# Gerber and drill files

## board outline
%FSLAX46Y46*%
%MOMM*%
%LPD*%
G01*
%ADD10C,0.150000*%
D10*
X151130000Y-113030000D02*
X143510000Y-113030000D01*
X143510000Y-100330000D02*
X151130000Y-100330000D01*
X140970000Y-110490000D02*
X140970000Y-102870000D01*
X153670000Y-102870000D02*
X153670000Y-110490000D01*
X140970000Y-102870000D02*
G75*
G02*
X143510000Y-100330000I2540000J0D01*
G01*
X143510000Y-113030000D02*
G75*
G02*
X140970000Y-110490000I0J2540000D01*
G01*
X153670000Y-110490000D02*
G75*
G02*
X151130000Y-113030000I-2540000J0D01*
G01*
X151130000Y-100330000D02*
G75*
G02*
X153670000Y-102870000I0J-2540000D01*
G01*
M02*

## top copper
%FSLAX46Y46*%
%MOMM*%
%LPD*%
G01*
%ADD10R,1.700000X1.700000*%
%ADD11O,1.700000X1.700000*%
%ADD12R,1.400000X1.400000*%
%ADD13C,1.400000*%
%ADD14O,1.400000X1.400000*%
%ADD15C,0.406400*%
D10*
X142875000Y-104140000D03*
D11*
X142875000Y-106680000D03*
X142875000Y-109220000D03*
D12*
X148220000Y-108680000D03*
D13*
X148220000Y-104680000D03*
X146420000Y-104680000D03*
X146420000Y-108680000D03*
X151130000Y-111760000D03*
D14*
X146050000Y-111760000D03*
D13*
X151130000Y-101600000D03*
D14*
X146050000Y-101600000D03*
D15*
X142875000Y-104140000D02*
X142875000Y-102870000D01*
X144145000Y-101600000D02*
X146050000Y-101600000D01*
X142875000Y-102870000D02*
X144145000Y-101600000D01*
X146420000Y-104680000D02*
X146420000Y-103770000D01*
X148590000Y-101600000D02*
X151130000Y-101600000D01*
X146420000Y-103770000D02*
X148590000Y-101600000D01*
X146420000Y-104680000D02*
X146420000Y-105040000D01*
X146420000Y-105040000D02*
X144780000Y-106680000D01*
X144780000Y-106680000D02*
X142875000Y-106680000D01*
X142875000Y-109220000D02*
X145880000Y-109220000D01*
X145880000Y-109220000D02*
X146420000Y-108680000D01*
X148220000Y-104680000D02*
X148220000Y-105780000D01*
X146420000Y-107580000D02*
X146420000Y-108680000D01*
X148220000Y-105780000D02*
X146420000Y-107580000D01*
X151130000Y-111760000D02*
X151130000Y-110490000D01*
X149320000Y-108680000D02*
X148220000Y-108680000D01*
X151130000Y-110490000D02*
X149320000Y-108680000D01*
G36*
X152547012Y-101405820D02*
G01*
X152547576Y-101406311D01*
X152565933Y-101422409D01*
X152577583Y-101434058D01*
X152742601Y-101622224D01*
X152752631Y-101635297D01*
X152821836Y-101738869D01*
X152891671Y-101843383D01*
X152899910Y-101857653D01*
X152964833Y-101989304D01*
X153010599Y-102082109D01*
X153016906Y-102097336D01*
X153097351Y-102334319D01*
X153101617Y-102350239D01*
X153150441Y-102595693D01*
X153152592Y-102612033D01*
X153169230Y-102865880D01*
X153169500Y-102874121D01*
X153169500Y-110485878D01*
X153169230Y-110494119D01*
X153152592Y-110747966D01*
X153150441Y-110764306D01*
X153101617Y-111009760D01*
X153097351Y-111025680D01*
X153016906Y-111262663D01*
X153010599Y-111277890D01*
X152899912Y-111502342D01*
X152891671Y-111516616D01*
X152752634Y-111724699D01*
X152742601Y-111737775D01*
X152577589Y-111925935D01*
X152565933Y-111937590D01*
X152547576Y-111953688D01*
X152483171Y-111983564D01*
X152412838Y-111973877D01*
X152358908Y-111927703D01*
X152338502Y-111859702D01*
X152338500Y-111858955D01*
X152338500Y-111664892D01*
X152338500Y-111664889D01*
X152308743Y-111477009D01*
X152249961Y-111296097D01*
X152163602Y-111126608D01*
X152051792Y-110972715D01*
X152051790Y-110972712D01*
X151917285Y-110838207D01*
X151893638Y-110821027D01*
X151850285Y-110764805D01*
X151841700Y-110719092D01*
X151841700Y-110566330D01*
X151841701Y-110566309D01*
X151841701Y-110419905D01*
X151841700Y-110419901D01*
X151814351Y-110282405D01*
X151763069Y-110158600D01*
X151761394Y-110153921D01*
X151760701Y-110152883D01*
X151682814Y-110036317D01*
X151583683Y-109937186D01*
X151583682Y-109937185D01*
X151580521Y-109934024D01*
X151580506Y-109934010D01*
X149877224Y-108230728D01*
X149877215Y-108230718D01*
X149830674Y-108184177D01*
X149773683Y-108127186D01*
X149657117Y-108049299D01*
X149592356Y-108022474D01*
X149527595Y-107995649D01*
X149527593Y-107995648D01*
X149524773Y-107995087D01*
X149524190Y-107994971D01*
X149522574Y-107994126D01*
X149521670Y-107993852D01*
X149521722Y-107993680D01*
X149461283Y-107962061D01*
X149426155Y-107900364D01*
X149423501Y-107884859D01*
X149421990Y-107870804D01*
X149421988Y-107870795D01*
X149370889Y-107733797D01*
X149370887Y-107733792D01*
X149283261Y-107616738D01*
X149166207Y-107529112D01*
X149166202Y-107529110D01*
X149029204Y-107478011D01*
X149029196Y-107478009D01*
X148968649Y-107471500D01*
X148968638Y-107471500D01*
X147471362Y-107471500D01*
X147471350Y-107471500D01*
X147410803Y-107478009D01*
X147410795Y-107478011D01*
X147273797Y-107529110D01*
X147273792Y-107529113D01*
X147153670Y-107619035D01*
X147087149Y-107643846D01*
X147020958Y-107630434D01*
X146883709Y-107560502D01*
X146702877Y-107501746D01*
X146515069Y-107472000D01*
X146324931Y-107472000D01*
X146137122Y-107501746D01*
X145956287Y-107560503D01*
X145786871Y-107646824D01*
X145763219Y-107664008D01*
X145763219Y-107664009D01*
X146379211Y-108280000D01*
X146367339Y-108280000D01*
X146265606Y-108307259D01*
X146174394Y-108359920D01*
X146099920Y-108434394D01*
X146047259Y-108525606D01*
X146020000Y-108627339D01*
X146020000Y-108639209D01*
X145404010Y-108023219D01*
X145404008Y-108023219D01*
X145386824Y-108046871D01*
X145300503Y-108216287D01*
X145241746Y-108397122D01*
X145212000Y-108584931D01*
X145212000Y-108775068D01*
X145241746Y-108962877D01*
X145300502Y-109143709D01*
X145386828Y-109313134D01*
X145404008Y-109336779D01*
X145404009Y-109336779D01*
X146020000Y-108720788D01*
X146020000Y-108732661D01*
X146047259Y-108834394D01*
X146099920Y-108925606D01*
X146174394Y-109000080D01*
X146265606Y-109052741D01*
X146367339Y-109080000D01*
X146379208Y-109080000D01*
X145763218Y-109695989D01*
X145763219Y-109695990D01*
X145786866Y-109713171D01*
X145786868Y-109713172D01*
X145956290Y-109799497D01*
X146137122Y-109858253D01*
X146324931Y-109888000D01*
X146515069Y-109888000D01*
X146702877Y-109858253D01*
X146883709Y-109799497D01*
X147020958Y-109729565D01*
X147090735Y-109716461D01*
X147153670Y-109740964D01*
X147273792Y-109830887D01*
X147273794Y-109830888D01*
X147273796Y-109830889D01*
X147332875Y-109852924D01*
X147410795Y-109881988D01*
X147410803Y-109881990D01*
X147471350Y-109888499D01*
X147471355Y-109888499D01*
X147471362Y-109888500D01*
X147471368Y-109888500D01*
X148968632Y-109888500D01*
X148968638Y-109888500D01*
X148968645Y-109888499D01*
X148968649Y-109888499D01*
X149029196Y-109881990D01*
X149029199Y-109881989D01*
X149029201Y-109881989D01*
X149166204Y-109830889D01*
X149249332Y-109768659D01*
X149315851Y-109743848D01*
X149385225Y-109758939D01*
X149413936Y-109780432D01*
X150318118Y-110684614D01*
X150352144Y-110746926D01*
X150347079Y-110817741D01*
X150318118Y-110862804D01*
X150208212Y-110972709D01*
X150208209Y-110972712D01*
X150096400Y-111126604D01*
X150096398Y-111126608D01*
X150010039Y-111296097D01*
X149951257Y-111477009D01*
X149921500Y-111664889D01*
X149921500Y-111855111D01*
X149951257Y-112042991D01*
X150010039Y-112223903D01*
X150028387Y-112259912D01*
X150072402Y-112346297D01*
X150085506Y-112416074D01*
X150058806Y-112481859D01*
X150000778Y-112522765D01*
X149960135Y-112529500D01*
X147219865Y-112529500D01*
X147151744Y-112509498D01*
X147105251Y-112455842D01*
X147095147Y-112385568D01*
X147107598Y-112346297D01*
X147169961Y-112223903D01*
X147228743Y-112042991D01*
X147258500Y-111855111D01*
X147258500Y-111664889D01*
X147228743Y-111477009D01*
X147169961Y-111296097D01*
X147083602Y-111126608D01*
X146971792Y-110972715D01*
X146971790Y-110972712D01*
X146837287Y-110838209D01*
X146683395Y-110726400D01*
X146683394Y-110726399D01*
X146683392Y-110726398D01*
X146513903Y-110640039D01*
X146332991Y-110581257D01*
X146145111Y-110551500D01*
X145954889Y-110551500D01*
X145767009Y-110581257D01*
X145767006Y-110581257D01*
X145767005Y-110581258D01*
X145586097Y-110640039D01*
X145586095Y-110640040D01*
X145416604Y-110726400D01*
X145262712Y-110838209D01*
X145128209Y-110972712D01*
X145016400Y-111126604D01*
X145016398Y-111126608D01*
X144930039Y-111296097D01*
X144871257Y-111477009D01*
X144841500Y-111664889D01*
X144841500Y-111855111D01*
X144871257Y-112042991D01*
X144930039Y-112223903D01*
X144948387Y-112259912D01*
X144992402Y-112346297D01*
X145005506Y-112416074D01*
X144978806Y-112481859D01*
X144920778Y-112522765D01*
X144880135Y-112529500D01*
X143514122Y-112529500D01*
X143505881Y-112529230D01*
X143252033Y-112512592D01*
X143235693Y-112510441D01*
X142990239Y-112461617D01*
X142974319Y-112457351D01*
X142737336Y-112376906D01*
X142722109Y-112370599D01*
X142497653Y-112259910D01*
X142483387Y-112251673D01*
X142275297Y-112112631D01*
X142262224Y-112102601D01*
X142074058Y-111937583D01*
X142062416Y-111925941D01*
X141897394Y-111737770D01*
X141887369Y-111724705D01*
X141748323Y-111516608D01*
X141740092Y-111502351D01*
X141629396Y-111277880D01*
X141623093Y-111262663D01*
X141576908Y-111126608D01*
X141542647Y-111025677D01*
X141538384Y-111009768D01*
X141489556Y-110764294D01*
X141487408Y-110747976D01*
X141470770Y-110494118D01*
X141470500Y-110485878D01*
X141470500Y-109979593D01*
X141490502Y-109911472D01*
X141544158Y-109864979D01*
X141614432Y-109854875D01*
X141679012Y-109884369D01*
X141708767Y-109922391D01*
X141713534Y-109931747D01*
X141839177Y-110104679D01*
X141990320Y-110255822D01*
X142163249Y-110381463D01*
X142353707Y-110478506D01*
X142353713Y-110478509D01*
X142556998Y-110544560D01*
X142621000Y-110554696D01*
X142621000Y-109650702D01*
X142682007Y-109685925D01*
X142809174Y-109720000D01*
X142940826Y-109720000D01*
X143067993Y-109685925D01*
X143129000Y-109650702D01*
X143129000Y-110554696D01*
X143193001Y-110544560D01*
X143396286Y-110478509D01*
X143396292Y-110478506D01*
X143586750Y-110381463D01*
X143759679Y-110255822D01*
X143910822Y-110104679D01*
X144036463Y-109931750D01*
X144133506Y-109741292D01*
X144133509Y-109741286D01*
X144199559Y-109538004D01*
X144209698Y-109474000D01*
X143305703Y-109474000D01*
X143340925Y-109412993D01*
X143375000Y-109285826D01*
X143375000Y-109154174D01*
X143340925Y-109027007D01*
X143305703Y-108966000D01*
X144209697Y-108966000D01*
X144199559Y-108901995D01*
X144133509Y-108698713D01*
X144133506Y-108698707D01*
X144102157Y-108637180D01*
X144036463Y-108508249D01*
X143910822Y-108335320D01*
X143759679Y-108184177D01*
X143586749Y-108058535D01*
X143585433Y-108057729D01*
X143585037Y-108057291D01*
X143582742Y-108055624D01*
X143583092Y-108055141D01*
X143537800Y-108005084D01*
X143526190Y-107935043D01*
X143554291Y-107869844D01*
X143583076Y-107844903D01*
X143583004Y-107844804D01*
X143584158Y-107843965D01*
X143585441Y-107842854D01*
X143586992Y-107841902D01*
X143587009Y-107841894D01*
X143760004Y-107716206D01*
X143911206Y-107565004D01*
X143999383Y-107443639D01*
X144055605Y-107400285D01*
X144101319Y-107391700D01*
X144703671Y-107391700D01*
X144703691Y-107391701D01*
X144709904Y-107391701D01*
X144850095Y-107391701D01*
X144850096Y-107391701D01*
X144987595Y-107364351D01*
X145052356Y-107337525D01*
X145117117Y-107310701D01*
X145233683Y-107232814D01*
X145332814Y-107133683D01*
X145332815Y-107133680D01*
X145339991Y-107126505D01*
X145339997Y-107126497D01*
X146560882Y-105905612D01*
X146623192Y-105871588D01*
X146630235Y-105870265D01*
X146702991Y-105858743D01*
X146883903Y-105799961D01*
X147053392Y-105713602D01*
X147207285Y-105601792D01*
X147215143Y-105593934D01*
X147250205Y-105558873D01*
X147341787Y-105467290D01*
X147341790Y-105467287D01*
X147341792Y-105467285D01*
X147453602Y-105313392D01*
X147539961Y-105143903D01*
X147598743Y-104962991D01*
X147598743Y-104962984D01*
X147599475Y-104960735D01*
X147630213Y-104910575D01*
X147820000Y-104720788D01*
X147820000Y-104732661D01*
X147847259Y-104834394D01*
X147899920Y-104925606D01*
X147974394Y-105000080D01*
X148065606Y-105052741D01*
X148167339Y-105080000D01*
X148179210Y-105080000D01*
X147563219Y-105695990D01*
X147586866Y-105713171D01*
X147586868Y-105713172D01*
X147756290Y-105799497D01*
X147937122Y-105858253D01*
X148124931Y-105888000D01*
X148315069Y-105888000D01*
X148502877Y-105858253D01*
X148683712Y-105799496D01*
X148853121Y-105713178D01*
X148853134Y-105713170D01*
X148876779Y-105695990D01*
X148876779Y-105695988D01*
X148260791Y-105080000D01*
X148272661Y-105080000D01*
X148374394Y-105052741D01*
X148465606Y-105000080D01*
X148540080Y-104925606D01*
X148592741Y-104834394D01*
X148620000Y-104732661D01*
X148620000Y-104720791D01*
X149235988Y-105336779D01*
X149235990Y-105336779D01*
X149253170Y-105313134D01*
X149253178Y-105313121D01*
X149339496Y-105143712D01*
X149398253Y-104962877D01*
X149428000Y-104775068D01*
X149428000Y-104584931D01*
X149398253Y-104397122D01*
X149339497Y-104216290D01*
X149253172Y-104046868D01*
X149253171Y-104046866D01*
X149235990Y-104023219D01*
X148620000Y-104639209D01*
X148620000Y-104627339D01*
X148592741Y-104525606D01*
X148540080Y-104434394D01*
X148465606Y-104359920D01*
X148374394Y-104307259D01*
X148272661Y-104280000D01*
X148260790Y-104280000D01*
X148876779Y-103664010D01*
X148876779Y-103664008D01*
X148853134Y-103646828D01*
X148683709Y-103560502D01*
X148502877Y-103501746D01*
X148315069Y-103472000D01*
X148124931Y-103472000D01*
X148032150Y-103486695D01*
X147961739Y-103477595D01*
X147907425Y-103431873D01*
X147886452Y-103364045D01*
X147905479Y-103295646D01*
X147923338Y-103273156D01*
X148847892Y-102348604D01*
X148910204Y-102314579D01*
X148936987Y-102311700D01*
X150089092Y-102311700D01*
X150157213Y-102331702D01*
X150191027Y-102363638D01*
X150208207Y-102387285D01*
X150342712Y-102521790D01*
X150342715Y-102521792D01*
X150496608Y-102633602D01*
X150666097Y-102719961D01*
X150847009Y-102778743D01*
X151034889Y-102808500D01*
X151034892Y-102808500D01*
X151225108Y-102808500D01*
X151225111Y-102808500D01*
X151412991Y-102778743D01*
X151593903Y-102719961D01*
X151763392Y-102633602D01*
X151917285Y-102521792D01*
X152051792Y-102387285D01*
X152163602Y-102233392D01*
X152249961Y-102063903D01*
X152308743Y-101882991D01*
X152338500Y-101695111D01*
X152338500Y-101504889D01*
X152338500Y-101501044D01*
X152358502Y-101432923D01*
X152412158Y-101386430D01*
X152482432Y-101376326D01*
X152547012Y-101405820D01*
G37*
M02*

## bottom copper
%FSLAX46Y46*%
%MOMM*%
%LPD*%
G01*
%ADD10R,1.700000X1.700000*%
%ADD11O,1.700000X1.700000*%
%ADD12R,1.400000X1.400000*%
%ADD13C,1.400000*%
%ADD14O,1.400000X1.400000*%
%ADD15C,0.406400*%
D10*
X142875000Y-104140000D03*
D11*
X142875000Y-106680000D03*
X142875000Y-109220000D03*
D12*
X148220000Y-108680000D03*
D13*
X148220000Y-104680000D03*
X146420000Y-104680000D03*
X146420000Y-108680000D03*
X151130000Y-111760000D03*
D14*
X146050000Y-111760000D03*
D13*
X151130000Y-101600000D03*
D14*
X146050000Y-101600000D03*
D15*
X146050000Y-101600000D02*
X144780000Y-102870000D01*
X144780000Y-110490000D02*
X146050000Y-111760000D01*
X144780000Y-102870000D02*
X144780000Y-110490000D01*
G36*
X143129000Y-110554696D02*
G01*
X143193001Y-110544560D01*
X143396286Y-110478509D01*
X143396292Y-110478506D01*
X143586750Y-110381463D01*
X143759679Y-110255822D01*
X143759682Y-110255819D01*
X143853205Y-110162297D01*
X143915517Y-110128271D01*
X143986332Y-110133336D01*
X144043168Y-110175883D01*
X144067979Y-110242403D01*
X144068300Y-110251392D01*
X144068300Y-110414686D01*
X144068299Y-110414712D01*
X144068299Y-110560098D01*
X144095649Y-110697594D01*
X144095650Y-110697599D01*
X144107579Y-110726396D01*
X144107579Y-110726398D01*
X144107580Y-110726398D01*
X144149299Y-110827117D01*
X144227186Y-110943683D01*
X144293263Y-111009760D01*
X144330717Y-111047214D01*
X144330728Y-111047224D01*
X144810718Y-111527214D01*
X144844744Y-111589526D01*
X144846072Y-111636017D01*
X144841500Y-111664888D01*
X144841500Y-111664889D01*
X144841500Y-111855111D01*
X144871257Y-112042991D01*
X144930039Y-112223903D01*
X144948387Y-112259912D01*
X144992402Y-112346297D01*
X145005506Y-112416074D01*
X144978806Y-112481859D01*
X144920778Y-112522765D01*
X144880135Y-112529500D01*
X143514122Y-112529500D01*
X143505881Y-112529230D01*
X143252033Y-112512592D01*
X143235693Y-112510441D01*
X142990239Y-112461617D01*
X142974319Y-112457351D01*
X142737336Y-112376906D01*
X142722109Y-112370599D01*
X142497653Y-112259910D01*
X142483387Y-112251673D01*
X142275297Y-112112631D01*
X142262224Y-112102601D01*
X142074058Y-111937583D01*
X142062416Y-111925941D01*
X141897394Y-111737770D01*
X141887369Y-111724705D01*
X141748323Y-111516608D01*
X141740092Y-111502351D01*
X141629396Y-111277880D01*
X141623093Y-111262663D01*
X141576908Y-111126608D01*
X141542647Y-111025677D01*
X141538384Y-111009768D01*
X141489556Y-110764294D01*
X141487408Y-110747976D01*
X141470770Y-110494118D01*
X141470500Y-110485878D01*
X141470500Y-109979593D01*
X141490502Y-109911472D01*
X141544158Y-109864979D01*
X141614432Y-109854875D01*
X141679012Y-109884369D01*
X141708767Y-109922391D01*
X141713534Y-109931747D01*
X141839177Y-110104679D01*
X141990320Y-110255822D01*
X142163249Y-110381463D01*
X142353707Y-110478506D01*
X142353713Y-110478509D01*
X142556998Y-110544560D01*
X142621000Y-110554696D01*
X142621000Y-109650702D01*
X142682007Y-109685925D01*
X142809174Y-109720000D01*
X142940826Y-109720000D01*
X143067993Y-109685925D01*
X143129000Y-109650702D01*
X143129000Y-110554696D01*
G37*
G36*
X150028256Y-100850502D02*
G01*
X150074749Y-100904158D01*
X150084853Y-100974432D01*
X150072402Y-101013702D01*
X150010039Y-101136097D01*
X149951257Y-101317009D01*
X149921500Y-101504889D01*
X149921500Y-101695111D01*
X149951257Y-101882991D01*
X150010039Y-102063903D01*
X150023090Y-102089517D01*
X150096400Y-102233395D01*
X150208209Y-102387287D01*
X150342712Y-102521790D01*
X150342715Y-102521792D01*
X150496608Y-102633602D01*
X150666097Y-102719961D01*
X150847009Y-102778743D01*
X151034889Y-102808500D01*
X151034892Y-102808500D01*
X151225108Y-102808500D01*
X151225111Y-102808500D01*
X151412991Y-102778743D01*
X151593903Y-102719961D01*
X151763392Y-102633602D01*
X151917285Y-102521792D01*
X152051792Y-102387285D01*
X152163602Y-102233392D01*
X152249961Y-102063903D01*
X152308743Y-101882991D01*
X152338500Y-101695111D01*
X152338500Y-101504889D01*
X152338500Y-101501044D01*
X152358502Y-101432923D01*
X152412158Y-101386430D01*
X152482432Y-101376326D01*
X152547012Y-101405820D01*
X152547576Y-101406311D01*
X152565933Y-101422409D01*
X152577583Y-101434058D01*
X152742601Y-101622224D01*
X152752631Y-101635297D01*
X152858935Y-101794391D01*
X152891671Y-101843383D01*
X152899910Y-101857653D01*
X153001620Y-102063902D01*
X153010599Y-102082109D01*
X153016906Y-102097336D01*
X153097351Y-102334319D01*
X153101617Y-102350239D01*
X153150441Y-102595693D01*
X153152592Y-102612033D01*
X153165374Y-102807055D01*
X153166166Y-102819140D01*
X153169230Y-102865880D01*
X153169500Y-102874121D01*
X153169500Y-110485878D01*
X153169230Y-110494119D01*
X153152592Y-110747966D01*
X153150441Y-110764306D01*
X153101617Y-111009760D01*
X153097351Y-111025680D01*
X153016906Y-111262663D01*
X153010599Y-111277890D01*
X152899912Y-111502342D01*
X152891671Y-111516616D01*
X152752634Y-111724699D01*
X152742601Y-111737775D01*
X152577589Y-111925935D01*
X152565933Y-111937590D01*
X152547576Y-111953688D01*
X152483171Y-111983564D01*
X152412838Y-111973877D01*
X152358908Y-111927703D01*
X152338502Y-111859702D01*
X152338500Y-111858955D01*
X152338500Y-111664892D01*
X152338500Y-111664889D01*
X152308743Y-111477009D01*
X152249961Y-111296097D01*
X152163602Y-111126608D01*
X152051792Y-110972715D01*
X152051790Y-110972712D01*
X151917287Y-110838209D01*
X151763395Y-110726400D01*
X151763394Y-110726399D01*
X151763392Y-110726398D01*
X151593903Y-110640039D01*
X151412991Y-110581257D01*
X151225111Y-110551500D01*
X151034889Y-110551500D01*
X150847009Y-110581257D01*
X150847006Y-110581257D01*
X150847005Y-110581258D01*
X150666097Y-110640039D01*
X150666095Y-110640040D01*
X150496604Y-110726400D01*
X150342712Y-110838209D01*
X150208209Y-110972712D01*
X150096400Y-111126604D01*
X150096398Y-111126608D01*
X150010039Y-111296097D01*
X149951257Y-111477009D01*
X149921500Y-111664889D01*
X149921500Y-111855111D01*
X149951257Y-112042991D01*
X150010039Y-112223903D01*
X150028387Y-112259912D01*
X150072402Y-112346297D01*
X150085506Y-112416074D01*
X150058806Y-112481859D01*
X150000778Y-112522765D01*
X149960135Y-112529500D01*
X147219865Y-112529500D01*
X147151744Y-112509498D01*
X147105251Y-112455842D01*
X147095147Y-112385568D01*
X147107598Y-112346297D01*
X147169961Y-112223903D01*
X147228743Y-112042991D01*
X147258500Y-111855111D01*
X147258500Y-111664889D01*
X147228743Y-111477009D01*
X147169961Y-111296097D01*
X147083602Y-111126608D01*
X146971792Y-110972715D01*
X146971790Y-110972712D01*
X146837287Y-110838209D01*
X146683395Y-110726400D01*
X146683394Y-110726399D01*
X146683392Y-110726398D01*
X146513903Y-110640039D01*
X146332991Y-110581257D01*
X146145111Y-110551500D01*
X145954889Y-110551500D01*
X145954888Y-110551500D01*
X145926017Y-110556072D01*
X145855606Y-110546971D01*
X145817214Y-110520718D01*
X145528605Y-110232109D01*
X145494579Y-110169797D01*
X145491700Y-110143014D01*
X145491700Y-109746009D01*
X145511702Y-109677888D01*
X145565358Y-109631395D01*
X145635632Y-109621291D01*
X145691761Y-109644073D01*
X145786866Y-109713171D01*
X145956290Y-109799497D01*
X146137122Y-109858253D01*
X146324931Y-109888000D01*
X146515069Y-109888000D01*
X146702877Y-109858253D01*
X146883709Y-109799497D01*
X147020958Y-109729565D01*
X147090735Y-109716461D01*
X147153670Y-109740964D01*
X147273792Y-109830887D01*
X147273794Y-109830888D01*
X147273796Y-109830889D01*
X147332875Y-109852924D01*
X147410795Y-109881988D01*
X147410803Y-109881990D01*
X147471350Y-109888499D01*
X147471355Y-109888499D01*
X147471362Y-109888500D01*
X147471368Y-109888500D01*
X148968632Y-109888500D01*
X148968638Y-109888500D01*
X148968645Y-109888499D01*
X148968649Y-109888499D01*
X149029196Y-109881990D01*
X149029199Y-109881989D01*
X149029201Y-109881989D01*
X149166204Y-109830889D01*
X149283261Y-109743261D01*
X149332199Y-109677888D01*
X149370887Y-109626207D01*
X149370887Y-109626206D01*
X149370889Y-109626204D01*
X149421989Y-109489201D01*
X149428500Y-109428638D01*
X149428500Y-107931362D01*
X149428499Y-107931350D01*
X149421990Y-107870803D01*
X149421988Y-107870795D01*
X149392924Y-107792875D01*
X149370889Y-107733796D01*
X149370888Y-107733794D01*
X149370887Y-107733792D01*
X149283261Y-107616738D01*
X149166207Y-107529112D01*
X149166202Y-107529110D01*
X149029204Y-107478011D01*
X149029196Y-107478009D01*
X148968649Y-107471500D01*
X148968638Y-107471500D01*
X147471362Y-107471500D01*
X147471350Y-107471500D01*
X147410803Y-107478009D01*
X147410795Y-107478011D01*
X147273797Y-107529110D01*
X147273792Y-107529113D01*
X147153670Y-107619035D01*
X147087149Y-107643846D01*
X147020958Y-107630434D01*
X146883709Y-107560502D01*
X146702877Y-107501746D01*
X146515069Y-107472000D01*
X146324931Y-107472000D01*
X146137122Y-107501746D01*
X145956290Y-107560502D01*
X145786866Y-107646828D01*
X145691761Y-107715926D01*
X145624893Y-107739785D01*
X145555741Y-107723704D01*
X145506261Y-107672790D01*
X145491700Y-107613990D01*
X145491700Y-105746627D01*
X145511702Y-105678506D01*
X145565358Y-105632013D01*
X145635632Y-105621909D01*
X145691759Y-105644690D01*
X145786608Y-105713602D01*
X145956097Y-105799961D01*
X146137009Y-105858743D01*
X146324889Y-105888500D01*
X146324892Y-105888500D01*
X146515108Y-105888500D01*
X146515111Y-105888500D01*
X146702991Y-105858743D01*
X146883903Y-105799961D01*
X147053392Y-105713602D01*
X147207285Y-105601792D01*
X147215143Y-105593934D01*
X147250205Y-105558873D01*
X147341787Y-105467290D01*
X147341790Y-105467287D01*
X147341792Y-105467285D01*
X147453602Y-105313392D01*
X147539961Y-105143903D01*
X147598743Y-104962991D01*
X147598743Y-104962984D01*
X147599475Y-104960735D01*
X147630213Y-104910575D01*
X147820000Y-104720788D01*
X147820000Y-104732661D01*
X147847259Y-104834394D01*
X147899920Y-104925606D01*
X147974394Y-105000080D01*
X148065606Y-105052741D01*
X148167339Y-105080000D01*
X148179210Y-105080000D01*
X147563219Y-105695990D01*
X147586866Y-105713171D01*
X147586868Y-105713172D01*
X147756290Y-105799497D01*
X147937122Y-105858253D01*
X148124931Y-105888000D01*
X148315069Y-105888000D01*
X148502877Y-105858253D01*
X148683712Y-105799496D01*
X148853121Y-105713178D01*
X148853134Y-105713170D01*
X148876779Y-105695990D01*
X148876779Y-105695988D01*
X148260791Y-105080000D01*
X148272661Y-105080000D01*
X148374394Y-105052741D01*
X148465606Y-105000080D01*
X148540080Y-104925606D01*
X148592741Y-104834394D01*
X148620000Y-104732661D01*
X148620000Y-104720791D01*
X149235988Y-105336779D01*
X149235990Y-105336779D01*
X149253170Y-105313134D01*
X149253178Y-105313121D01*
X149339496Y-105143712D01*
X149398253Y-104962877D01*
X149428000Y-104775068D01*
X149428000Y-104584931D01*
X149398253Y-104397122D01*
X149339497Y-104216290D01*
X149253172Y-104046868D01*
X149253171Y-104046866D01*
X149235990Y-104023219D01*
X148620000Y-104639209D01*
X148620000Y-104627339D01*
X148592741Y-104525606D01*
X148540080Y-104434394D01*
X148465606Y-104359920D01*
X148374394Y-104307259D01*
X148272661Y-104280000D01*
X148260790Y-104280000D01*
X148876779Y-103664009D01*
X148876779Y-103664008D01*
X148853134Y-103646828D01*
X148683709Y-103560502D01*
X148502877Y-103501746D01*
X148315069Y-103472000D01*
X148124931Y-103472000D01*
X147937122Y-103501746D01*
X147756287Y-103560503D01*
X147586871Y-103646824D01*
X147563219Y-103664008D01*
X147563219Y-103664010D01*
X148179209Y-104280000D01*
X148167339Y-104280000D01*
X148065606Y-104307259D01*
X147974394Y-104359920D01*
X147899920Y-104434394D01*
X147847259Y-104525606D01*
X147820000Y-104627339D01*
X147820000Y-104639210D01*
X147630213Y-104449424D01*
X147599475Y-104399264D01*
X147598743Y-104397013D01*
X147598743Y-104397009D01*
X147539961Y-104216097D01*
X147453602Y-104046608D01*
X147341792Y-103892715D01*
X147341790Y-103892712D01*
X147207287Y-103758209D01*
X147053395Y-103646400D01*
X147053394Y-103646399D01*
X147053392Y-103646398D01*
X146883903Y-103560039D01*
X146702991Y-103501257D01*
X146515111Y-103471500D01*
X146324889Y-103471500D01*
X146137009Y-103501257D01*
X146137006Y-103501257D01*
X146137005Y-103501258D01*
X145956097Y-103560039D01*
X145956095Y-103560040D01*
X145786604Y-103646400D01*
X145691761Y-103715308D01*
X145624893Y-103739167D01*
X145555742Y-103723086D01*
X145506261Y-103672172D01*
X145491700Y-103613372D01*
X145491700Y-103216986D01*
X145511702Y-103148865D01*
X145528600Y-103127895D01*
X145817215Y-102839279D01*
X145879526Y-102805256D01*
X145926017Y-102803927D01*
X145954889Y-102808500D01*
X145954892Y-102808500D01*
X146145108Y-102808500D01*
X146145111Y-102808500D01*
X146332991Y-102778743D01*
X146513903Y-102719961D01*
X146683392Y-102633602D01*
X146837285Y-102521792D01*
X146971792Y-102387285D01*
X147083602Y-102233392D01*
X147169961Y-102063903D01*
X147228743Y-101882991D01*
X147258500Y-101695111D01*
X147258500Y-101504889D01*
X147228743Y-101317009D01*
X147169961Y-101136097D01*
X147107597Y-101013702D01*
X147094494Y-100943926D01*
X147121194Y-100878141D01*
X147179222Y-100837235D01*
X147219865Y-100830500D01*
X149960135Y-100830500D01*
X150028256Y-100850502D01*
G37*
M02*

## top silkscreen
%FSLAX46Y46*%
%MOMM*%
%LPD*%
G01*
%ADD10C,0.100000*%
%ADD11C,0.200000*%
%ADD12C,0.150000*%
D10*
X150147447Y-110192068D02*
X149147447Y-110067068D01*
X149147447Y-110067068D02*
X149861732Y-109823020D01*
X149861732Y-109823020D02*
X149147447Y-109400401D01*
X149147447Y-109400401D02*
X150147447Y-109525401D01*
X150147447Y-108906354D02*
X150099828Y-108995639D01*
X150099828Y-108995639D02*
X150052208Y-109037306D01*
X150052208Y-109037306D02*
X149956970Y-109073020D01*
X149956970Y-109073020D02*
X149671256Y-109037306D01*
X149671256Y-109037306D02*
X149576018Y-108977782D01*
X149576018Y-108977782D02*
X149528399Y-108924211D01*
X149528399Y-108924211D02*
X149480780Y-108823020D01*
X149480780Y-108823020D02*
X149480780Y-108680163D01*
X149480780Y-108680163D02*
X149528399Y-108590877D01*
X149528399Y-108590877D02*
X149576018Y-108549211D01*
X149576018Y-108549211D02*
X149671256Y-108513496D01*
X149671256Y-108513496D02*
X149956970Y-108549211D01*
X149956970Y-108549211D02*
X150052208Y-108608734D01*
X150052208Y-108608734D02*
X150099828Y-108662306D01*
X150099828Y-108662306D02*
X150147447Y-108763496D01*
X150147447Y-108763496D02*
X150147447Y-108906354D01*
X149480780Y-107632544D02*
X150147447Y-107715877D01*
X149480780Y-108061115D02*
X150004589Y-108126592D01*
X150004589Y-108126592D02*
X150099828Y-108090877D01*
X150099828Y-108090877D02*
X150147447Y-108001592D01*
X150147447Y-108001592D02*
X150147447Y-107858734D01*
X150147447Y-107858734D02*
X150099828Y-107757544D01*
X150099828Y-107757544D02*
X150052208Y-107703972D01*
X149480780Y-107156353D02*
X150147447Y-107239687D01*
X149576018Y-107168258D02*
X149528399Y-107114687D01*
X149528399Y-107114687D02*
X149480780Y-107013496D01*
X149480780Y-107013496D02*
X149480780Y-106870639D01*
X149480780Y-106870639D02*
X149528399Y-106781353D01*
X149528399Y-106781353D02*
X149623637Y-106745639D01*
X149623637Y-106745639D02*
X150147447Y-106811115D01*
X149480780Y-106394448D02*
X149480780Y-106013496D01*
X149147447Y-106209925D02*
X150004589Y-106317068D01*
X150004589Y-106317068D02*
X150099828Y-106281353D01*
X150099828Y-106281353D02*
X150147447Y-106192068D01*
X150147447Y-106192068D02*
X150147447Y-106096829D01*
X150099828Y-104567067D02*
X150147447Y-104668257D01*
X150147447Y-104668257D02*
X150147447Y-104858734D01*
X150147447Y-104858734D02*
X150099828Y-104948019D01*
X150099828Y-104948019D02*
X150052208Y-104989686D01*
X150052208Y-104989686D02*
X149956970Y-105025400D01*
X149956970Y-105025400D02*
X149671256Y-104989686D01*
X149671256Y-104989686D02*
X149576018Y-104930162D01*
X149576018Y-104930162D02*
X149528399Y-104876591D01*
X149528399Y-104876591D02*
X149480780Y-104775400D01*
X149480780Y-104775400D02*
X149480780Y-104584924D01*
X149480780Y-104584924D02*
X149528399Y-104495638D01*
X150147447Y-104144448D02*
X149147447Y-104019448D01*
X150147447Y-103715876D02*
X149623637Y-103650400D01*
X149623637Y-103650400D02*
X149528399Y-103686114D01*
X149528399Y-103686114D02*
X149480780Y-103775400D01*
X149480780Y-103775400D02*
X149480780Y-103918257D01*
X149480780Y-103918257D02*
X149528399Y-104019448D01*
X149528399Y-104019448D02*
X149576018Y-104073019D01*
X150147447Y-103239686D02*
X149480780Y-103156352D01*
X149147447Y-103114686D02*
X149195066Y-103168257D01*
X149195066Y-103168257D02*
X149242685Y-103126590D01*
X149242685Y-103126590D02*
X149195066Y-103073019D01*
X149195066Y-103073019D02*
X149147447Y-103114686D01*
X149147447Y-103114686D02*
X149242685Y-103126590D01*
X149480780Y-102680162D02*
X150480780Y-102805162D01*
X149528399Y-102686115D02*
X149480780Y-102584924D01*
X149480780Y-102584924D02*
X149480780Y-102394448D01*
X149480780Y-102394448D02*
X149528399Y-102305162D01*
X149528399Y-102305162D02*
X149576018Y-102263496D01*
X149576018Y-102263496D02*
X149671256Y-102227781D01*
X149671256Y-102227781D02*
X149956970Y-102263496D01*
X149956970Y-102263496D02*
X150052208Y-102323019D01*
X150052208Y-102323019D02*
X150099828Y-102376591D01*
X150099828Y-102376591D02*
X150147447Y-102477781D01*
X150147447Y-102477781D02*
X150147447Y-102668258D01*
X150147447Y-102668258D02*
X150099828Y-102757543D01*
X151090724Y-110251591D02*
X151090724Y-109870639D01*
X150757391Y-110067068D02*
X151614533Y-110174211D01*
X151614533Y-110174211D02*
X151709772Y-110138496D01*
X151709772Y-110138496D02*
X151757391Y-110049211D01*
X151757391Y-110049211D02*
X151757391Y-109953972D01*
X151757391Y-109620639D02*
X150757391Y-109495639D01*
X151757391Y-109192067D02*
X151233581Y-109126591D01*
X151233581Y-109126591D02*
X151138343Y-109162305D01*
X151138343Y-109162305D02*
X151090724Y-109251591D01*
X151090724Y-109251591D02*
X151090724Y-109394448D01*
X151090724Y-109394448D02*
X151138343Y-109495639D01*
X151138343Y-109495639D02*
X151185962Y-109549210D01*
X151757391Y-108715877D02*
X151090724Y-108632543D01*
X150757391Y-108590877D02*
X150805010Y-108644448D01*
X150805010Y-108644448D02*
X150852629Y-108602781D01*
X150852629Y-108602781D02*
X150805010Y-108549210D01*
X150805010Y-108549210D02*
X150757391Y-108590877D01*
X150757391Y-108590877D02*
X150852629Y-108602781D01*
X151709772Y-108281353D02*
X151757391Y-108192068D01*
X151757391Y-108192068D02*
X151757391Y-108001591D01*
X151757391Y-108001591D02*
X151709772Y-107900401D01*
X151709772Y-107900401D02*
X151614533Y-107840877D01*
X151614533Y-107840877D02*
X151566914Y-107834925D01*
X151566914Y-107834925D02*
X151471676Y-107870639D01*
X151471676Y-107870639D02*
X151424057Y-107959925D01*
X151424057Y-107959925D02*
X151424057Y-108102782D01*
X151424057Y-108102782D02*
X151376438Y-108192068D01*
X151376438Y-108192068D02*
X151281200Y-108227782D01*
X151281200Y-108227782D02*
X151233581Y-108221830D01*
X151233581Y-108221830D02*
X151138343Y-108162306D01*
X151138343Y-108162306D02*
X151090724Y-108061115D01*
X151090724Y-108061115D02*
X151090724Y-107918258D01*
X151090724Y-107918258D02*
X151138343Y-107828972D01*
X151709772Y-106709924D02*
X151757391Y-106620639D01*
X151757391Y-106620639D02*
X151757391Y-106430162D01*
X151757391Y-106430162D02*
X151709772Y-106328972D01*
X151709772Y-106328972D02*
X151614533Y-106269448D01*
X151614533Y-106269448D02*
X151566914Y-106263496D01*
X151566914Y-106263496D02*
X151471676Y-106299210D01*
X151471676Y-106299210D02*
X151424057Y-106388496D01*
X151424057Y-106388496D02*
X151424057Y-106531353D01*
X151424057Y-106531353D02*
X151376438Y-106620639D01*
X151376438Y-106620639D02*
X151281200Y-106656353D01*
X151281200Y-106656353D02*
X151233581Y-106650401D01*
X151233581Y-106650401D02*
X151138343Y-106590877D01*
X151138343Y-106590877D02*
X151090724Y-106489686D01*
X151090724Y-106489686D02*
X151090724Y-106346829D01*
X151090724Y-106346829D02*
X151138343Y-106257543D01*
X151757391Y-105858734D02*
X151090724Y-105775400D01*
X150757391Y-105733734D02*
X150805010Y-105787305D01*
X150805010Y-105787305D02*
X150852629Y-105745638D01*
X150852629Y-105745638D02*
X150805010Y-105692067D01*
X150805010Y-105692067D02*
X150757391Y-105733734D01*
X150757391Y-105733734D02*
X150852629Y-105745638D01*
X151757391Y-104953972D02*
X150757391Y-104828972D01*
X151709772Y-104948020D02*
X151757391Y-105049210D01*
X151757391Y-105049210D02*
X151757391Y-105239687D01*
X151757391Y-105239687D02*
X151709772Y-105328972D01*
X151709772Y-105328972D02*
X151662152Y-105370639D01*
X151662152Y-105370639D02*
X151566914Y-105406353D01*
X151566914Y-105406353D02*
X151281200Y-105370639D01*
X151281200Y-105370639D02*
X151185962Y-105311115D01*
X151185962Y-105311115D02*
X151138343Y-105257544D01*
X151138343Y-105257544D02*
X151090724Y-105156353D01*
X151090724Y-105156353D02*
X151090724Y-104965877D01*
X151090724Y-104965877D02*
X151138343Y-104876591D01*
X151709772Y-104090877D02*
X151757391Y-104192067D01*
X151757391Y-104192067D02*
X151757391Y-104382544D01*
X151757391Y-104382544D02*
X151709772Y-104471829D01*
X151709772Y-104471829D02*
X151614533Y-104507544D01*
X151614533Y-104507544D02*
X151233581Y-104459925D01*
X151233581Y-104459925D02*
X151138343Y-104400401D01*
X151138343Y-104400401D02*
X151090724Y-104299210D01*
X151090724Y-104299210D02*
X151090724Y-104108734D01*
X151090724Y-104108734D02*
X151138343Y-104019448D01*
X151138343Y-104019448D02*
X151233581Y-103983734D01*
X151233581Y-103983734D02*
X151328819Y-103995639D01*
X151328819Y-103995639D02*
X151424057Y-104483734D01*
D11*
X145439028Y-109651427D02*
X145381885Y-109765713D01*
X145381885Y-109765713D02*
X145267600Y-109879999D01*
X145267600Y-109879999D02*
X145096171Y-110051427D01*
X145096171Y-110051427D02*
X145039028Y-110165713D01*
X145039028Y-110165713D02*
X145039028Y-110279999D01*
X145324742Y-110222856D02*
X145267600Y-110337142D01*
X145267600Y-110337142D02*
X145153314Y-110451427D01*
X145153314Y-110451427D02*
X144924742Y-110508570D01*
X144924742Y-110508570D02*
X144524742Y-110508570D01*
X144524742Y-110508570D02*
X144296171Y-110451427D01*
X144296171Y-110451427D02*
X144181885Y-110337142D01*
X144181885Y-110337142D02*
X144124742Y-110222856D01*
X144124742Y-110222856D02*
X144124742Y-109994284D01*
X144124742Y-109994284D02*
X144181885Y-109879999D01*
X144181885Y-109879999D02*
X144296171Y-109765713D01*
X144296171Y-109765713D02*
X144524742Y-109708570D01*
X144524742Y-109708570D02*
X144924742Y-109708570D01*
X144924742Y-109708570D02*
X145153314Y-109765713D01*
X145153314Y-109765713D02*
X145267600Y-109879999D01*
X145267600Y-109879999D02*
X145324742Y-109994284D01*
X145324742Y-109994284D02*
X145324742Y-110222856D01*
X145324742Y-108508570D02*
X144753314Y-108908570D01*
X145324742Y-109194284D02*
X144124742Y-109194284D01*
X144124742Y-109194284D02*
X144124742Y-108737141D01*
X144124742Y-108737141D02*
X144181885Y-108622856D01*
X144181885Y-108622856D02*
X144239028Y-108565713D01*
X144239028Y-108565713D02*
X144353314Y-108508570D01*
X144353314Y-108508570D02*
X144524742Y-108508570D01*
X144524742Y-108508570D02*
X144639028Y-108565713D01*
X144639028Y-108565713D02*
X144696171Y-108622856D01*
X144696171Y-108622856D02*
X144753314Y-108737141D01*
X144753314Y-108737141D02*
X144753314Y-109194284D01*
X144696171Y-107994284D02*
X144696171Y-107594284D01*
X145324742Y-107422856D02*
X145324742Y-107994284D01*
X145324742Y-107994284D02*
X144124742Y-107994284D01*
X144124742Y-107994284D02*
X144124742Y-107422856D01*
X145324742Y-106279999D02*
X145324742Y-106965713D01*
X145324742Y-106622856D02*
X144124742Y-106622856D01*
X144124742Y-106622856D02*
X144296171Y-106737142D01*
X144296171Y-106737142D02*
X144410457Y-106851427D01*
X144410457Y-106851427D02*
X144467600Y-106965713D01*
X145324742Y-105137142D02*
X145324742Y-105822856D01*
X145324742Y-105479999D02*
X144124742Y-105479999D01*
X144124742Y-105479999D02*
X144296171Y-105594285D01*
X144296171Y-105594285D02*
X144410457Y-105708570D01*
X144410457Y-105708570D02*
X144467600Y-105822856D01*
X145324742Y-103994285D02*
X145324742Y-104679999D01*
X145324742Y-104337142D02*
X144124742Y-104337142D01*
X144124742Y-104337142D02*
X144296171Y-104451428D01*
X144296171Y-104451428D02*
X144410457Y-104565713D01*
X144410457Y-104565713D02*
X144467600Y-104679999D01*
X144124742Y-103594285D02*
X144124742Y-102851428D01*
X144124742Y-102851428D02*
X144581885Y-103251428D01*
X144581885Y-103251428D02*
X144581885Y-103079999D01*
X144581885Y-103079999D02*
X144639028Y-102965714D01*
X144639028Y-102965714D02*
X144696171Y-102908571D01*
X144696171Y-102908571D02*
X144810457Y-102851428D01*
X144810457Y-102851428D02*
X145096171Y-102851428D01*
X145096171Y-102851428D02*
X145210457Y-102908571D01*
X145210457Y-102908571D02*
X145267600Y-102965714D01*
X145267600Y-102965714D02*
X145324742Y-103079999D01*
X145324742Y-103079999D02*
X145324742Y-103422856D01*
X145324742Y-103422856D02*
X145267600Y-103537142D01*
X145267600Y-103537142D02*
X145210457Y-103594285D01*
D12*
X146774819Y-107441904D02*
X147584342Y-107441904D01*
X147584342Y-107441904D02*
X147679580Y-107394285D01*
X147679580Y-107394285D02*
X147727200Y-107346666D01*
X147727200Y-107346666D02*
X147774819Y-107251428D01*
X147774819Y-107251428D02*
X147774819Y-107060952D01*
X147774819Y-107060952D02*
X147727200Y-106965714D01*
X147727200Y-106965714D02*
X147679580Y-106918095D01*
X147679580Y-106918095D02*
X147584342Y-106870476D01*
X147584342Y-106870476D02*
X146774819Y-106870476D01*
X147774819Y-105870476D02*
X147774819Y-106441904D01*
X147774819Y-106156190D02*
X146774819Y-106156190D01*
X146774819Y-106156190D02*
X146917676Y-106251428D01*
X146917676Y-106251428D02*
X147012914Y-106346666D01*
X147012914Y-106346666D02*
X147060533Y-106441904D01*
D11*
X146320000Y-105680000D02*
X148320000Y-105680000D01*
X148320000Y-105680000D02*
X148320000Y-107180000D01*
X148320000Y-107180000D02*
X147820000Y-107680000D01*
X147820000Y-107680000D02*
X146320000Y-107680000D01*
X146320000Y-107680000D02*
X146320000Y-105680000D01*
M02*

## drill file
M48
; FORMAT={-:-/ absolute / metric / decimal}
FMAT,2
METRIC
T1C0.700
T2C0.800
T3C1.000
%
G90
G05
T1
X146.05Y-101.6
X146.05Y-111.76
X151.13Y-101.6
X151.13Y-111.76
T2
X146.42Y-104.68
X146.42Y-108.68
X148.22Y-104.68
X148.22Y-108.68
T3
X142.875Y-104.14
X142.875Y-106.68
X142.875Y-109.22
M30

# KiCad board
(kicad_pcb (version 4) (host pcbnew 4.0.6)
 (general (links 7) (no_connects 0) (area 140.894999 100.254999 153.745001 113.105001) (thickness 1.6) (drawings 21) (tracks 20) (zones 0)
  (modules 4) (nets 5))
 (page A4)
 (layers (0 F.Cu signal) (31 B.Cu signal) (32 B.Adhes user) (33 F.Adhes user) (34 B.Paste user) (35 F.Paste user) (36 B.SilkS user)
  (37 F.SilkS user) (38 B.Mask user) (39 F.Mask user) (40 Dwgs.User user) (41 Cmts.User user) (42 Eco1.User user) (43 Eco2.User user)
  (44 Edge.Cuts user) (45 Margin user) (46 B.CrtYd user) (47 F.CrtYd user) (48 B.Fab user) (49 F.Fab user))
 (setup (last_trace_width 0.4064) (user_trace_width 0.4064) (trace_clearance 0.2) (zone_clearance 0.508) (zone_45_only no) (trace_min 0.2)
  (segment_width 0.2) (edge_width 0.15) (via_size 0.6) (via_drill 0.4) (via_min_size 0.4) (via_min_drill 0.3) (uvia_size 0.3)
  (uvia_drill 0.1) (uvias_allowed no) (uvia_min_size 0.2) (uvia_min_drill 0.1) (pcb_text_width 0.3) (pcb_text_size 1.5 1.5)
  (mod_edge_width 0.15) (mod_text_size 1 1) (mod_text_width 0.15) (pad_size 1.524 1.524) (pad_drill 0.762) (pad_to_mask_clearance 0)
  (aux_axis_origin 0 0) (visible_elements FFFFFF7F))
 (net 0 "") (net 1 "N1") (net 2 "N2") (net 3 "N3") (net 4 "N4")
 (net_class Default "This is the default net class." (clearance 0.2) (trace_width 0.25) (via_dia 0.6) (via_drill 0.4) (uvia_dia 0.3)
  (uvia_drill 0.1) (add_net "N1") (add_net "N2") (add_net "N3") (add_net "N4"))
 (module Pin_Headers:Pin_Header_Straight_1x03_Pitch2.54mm (layer B.Cu) (at 142.875 104.14 180)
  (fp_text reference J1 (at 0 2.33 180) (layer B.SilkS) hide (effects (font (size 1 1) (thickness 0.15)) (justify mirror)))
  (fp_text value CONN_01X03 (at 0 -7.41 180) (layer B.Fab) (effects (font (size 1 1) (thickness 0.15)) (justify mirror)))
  (pad 1 thru_hole rect (at 0 0 180) (size 1.7 1.7) (drill 1) (layers *.Cu *.Mask) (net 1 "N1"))
  (pad 2 thru_hole oval (at 0 -2.54 180) (size 1.7 1.7) (drill 1) (layers *.Cu *.Mask) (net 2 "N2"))
  (pad 3 thru_hole oval (at 0 -5.08 180) (size 1.7 1.7) (drill 1) (layers *.Cu *.Mask) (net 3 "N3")))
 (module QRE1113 (layer F.Cu) (at 147.32 106.68 90)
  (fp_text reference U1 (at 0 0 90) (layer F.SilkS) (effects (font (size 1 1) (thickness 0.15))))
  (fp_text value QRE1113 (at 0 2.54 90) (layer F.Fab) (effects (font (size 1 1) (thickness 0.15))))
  (fp_line (start 1 -1) (end 1 1) (layer F.SilkS) (width 0.2))
  (fp_line (start 1 1) (end -0.5 1) (layer F.SilkS) (width 0.2))
  (fp_line (start -0.5 1) (end -1 0.5) (layer F.SilkS) (width 0.2))
  (fp_line (start -1 0.5) (end -1 -1) (layer F.SilkS) (width 0.2))
  (fp_line (start -1 -1) (end 1 -1) (layer F.SilkS) (width 0.2))
  (pad 1 thru_hole rect (at -2 0.9 90) (size 1.4 1.4) (drill 0.8) (layers *.Cu *.Mask) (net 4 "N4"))
  (pad 2 thru_hole circle (at 2 0.9 90) (size 1.4 1.4) (drill 0.8) (layers *.Cu *.Mask) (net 3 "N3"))
  (pad 3 thru_hole circle (at 2 -0.9 90) (size 1.4 1.4) (drill 0.8) (layers *.Cu *.Mask) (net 2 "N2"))
  (pad 4 thru_hole circle (at -2 -0.9 90) (size 1.4 1.4) (drill 0.8) (layers *.Cu *.Mask) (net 3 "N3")))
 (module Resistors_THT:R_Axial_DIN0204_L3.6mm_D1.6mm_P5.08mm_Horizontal (layer B.Cu) (at 151.13 111.76 180)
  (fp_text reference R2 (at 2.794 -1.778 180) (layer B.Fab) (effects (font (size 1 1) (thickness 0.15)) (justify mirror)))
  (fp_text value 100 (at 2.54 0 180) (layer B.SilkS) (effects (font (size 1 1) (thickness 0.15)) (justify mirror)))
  (pad 1 thru_hole circle (at 0 0 180) (size 1.4 1.4) (drill 0.7) (layers *.Cu *.Mask) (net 4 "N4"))
  (pad 2 thru_hole oval (at 5.08 0 180) (size 1.4 1.4) (drill 0.7) (layers *.Cu *.Mask) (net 1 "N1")))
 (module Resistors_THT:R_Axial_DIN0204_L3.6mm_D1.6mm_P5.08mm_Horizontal (layer B.Cu) (at 151.13 101.6 180)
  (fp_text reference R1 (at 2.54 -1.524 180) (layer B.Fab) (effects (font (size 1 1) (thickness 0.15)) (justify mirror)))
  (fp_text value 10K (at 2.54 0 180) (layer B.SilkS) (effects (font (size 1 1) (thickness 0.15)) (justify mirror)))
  (pad 1 thru_hole circle (at 0 0 180) (size 1.4 1.4) (drill 0.7) (layers *.Cu *.Mask) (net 2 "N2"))
  (pad 2 thru_hole oval (at 5.08 0 180) (size 1.4 1.4) (drill 0.7) (layers *.Cu *.Mask) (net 1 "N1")))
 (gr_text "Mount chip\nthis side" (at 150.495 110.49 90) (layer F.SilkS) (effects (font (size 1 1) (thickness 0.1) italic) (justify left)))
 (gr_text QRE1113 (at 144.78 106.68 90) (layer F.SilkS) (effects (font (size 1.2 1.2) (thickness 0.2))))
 (gr_line (start 151.13 113.03) (end 143.51 113.03) (angle 90) (layer Edge.Cuts) (width 0.15))
 (gr_line (start 143.51 100.33) (end 151.13 100.33) (angle 90) (layer Edge.Cuts) (width 0.15))
 (gr_line (start 140.97 110.49) (end 140.97 102.87) (angle 90) (layer Edge.Cuts) (width 0.15))
 (gr_line (start 153.67 102.87) (end 153.67 110.49) (angle 90) (layer Edge.Cuts) (width 0.15))
 (gr_arc (start 143.51 102.87) (end 140.97 102.87) (angle 90) (layer Edge.Cuts) (width 0.15))
 (gr_arc (start 143.51 110.49) (end 143.51 113.03) (angle 90) (layer Edge.Cuts) (width 0.15))
 (gr_arc (start 151.13 110.49) (end 153.67 110.49) (angle 90) (layer Edge.Cuts) (width 0.15))
 (gr_arc (start 151.13 102.87) (end 151.13 100.33) (angle 90) (layer Edge.Cuts) (width 0.15))
 (segment (start 146.05 101.6) (end 144.78 102.87) (width 0.4064) (layer B.Cu) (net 1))
 (segment (start 144.78 110.49) (end 146.05 111.76) (width 0.4064) (layer B.Cu) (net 1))
 (segment (start 144.78 102.87) (end 144.78 110.49) (width 0.4064) (layer B.Cu) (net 1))
 (segment (start 142.875 104.14) (end 142.875 102.87) (width 0.4064) (layer F.Cu) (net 1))
 (segment (start 144.145 101.6) (end 146.05 101.6) (width 0.4064) (layer F.Cu) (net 1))
 (segment (start 142.875 102.87) (end 144.145 101.6) (width 0.4064) (layer F.Cu) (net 1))
 (segment (start 146.42 104.68) (end 146.42 103.77) (width 0.4064) (layer F.Cu) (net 2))
 (segment (start 148.59 101.6) (end 151.13 101.6) (width 0.4064) (layer F.Cu) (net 2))
 (segment (start 146.42 103.77) (end 148.59 101.6) (width 0.4064) (layer F.Cu) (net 2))
 (segment (start 146.42 104.68) (end 146.42 105.04) (width 0.4064) (layer F.Cu) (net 2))
 (segment (start 146.42 105.04) (end 144.78 106.68) (width 0.4064) (layer F.Cu) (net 2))
 (segment (start 144.78 106.68) (end 142.875 106.68) (width 0.4064) (layer F.Cu) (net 2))
 (segment (start 142.875 109.22) (end 145.88 109.22) (width 0.4064) (layer F.Cu) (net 3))
 (segment (start 145.88 109.22) (end 146.42 108.68) (width 0.4064) (layer F.Cu) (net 3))
 (segment (start 148.22 104.68) (end 148.22 105.78) (width 0.4064) (layer F.Cu) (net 3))
 (segment (start 146.42 107.58) (end 146.42 108.68) (width 0.4064) (layer F.Cu) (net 3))
 (segment (start 148.22 105.78) (end 146.42 107.58) (width 0.4064) (layer F.Cu) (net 3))
 (segment (start 151.13 111.76) (end 151.13 110.49) (width 0.4064) (layer F.Cu) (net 4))
 (segment (start 149.32 108.68) (end 148.22 108.68) (width 0.4064) (layer F.Cu) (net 4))
 (segment (start 151.13 110.49) (end 149.32 108.68) (width 0.4064) (layer F.Cu) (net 4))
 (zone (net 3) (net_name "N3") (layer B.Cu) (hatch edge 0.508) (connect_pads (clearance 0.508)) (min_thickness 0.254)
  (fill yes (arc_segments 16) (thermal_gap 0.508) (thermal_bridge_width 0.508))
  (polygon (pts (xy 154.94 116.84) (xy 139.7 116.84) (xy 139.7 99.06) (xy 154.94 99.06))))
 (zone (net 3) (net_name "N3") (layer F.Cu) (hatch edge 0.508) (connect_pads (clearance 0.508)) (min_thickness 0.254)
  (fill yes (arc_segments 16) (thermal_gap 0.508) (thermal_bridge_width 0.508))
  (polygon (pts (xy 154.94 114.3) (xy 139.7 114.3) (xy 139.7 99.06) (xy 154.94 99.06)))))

